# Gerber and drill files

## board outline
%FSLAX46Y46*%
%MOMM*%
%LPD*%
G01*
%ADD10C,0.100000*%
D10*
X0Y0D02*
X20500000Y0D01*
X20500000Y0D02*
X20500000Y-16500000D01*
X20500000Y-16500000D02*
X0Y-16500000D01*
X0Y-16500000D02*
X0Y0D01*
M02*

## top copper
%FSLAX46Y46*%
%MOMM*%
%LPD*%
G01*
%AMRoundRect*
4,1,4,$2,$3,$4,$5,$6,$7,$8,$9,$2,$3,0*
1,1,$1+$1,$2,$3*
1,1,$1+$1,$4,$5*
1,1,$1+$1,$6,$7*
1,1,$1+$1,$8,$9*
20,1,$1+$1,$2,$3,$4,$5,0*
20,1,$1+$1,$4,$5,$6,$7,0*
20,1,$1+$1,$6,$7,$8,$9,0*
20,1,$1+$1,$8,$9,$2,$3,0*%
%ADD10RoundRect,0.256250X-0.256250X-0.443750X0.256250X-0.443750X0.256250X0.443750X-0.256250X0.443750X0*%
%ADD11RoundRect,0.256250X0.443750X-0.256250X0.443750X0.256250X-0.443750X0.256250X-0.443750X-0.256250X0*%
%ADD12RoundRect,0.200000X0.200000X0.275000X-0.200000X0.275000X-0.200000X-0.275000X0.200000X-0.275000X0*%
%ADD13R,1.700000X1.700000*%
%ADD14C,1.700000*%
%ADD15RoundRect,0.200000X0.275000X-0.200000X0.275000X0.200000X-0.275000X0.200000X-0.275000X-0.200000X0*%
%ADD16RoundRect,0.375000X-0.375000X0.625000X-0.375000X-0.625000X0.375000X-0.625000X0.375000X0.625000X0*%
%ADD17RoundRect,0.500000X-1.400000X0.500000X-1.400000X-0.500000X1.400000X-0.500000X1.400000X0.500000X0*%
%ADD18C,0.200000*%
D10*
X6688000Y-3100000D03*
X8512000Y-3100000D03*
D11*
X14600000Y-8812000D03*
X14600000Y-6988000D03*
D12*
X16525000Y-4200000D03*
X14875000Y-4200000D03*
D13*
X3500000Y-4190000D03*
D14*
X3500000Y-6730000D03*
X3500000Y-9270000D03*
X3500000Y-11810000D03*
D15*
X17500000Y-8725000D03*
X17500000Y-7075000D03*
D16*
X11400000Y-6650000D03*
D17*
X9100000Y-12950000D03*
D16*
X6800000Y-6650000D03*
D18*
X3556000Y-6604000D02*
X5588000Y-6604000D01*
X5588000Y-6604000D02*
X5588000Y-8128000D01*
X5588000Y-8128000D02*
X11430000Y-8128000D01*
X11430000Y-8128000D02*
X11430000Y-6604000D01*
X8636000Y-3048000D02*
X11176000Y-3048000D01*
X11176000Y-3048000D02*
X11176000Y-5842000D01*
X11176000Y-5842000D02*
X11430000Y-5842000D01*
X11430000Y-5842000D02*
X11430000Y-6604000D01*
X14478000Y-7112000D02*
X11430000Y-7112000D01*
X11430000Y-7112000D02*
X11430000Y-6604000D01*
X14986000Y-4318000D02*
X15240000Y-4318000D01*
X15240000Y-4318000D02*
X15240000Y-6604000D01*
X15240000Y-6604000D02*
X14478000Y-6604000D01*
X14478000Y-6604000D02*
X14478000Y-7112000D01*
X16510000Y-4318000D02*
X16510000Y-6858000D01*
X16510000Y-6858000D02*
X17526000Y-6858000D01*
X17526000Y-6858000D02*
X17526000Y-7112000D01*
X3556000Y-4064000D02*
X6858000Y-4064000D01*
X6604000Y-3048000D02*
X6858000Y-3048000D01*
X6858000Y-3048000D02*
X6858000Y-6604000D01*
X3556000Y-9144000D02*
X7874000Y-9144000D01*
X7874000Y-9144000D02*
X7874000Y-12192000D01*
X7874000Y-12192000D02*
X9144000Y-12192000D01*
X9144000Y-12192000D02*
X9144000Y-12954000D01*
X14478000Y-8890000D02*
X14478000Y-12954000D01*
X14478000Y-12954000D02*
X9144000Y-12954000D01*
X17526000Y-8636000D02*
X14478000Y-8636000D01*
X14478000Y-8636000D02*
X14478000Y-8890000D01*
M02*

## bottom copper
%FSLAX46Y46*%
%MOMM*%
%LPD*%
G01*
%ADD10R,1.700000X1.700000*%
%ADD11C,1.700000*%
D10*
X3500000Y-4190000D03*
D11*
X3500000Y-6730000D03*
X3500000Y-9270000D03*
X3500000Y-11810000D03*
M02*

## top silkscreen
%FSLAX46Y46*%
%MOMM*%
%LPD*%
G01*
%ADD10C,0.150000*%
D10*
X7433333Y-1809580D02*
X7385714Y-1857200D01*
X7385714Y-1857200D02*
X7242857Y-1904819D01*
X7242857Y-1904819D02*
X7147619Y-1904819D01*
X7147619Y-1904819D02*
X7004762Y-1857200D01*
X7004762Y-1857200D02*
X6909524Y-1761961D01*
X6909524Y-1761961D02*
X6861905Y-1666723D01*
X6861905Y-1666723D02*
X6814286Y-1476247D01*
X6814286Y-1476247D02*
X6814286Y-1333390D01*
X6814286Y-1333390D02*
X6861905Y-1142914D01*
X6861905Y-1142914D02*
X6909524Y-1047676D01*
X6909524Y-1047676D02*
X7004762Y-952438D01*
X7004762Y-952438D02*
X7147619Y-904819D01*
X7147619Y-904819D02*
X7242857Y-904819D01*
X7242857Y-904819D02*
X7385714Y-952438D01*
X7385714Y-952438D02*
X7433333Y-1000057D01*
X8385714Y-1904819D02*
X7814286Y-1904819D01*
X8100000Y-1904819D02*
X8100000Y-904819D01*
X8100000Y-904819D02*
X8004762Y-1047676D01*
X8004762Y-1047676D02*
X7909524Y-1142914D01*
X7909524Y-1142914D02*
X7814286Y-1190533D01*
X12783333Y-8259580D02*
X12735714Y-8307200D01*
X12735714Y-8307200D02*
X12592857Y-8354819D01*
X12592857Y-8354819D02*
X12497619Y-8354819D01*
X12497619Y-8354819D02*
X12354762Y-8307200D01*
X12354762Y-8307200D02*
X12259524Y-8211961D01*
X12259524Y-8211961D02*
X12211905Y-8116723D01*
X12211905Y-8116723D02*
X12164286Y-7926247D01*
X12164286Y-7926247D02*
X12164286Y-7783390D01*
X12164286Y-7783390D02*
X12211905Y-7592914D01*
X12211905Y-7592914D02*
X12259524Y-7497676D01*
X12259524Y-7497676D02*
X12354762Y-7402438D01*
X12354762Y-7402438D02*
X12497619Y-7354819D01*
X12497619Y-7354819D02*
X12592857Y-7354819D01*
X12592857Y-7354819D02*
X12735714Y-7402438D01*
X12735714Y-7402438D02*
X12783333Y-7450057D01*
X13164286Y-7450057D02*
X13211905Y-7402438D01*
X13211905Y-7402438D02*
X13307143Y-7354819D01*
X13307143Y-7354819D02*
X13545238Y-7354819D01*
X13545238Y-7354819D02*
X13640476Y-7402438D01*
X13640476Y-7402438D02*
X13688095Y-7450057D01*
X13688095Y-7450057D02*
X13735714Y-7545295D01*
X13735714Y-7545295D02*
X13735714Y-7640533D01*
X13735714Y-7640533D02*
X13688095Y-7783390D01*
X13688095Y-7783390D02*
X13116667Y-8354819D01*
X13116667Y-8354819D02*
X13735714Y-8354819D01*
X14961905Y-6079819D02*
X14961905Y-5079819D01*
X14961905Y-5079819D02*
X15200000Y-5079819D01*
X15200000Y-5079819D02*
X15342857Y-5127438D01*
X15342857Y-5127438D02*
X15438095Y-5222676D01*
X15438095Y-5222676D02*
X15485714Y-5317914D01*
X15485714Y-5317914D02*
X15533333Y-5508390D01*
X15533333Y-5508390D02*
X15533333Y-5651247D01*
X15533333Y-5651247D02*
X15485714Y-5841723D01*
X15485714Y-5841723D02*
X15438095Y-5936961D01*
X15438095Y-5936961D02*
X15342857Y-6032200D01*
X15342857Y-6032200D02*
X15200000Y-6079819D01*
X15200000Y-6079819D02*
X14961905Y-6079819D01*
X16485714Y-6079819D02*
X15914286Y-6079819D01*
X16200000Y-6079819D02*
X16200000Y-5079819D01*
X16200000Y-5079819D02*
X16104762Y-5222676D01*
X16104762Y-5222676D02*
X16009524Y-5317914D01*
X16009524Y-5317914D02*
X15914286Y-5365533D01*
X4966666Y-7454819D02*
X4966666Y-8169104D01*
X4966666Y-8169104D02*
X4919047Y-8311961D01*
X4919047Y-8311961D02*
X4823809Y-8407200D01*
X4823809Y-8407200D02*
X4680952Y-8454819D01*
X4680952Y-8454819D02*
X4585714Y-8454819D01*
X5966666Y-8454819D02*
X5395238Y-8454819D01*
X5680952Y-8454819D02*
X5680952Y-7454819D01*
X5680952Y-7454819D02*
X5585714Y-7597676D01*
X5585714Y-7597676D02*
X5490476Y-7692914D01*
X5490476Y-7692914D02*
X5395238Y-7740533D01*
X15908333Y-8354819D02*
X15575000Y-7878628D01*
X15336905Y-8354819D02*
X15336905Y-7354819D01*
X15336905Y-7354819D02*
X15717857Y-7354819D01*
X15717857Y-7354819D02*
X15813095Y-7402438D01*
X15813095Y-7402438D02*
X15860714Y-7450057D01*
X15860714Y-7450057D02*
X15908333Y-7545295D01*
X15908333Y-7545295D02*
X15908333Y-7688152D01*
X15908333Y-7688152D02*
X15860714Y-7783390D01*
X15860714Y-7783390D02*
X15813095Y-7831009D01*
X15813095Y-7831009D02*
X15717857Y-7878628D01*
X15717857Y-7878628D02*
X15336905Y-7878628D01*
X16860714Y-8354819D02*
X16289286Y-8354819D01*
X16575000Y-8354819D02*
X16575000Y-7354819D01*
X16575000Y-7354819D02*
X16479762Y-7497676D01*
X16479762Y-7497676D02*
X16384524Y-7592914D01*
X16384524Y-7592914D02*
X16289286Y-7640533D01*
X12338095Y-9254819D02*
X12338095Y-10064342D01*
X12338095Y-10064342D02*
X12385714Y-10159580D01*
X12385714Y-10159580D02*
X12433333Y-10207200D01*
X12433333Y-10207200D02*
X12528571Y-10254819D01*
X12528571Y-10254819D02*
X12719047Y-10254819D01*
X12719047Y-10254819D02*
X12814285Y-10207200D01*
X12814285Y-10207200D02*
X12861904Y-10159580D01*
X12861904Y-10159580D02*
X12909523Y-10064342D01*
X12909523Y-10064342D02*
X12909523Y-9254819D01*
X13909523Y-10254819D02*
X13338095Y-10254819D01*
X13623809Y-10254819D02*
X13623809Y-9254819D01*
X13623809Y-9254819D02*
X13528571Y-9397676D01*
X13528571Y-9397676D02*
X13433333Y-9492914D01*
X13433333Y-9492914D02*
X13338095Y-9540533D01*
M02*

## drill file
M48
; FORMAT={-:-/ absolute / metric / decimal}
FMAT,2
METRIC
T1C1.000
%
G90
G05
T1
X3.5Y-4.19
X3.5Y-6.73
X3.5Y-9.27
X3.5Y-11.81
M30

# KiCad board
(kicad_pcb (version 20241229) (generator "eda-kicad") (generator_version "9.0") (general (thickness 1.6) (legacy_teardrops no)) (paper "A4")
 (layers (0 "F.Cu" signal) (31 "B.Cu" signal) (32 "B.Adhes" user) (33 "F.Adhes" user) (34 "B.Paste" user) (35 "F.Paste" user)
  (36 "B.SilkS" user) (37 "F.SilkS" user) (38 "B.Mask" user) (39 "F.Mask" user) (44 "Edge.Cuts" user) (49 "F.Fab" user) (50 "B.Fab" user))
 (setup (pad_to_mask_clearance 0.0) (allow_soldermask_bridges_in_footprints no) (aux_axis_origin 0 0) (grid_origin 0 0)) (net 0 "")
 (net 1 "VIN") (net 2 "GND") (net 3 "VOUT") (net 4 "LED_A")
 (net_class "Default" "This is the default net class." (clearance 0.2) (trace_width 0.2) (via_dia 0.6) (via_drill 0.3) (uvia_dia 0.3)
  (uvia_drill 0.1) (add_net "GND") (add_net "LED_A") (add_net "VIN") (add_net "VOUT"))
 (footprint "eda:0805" (layer "F.Cu") (at 7.6 3.1 0)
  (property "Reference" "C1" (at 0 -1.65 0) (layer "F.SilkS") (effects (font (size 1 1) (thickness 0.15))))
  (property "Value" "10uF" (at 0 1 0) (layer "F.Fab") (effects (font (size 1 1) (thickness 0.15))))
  (pad "1" smd roundrect (at -0.912 0 0) (size 1.025 1.4) (roundrect_rratio 0.25) (layers "F.Cu" "F.Paste" "F.Mask") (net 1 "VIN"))
  (pad "2" smd roundrect (at 0.912 0 0) (size 1.025 1.4) (roundrect_rratio 0.25) (layers "F.Cu" "F.Paste" "F.Mask") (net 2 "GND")))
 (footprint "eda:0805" (layer "F.Cu") (at 14.6 7.9 -270)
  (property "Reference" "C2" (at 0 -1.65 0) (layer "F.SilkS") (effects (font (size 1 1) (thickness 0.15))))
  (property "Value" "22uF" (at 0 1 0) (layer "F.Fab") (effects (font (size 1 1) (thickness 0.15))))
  (pad "1" smd roundrect (at -0.912 0 -270) (size 1.025 1.4) (roundrect_rratio 0.25) (layers "F.Cu" "F.Paste" "F.Mask") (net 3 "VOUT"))
  (pad "2" smd roundrect (at 0.912 0 -270) (size 1.025 1.4) (roundrect_rratio 0.25) (layers "F.Cu" "F.Paste" "F.Mask") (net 2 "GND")))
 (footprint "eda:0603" (layer "F.Cu") (at 15.7 4.2 -180)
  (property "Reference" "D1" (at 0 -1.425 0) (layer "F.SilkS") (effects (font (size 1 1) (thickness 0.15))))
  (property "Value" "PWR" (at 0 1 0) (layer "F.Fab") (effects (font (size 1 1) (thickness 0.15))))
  (pad "1" smd roundrect (at -0.825 0 -180) (size 0.8 0.95) (roundrect_rratio 0.25) (layers "F.Cu" "F.Paste" "F.Mask") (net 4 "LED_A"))
  (pad "2" smd roundrect (at 0.825 0 -180) (size 0.8 0.95) (roundrect_rratio 0.25) (layers "F.Cu" "F.Paste" "F.Mask") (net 2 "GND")))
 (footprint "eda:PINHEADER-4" (layer "F.Cu") (at 3.5 8 -90)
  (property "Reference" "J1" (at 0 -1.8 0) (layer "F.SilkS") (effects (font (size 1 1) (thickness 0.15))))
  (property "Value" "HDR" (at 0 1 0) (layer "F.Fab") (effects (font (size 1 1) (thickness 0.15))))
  (pad "1" thru_hole rect (at -3.81 0 -90) (size 1.7 1.7) (drill 1) (layers "*.Cu" "*.Mask") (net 1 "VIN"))
  (pad "2" thru_hole circle (at -1.27 0 -90) (size 1.7 1.7) (drill 1) (layers "*.Cu" "*.Mask") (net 2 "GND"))
  (pad "3" thru_hole circle (at 1.27 0 -90) (size 1.7 1.7) (drill 1) (layers "*.Cu" "*.Mask") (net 3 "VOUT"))
  (pad "4" thru_hole circle (at 3.81 0 -90) (size 1.7 1.7) (drill 1) (layers "*.Cu" "*.Mask")))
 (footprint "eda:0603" (layer "F.Cu") (at 17.5 7.9 -270)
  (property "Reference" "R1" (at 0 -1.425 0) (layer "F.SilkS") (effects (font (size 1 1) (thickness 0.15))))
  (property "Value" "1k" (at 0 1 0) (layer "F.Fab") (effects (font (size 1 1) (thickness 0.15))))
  (pad "1" smd roundrect (at -0.825 0 -270) (size 0.8 0.95) (roundrect_rratio 0.25) (layers "F.Cu" "F.Paste" "F.Mask") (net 3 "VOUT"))
  (pad "2" smd roundrect (at 0.825 0 -270) (size 0.8 0.95) (roundrect_rratio 0.25) (layers "F.Cu" "F.Paste" "F.Mask") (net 4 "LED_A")))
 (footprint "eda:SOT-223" (layer "F.Cu") (at 9.1 9.8 -90)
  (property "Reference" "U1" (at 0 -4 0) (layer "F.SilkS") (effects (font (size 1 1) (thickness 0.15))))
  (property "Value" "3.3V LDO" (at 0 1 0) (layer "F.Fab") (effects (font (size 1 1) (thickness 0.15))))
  (pad "1" smd roundrect (at -3.15 -2.3 -90) (size 2 1.5) (roundrect_rratio 0.25) (layers "F.Cu" "F.Paste" "F.Mask") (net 2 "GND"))
  (pad "2" smd roundrect (at 3.15 0 -90) (size 2 3.8) (roundrect_rratio 0.25) (layers "F.Cu" "F.Paste" "F.Mask") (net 3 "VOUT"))
  (pad "3" smd roundrect (at -3.15 2.3 -90) (size 2 1.5) (roundrect_rratio 0.25) (layers "F.Cu" "F.Paste" "F.Mask") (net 1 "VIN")))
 (segment (start 3.556 6.604) (end 5.588 6.604) (width 0.2) (layer "F.Cu") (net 2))
 (segment (start 5.588 6.604) (end 5.588 8.128) (width 0.2) (layer "F.Cu") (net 2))
 (segment (start 5.588 8.128) (end 11.43 8.128) (width 0.2) (layer "F.Cu") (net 2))
 (segment (start 11.43 8.128) (end 11.43 6.604) (width 0.2) (layer "F.Cu") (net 2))
 (segment (start 8.636 3.048) (end 11.176 3.048) (width 0.2) (layer "F.Cu") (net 2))
 (segment (start 11.176 3.048) (end 11.176 5.842) (width 0.2) (layer "F.Cu") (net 2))
 (segment (start 11.176 5.842) (end 11.43 5.842) (width 0.2) (layer "F.Cu") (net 2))
 (segment (start 11.43 5.842) (end 11.43 6.604) (width 0.2) (layer "F.Cu") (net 2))
 (segment (start 14.478 7.112) (end 11.43 7.112) (width 0.2) (layer "F.Cu") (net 2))
 (segment (start 11.43 7.112) (end 11.43 6.604) (width 0.2) (layer "F.Cu") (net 2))
 (segment (start 14.986 4.318) (end 15.24 4.318) (width 0.2) (layer "F.Cu") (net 2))
 (segment (start 15.24 4.318) (end 15.24 6.604) (width 0.2) (layer "F.Cu") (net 2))
 (segment (start 15.24 6.604) (end 14.478 6.604) (width 0.2) (layer "F.Cu") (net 2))
 (segment (start 14.478 6.604) (end 14.478 7.112) (width 0.2) (layer "F.Cu") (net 2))
 (segment (start 16.51 4.318) (end 16.51 6.858) (width 0.2) (layer "F.Cu") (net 4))
 (segment (start 16.51 6.858) (end 17.526 6.858) (width 0.2) (layer "F.Cu") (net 4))
 (segment (start 17.526 6.858) (end 17.526 7.112) (width 0.2) (layer "F.Cu") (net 4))
 (segment (start 3.556 4.064) (end 6.858 4.064) (width 0.2) (layer "F.Cu") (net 1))
 (segment (start 6.604 3.048) (end 6.858 3.048) (width 0.2) (layer "F.Cu") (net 1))
 (segment (start 6.858 3.048) (end 6.858 6.604) (width 0.2) (layer "F.Cu") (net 1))
 (segment (start 3.556 9.144) (end 7.874 9.144) (width 0.2) (layer "F.Cu") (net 3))
 (segment (start 7.874 9.144) (end 7.874 12.192) (width 0.2) (layer "F.Cu") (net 3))
 (segment (start 7.874 12.192) (end 9.144 12.192) (width 0.2) (layer "F.Cu") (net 3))
 (segment (start 9.144 12.192) (end 9.144 12.954) (width 0.2) (layer "F.Cu") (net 3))
 (segment (start 14.478 8.89) (end 14.478 12.954) (width 0.2) (layer "F.Cu") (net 3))
 (segment (start 14.478 12.954) (end 9.144 12.954) (width 0.2) (layer "F.Cu") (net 3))
 (segment (start 17.526 8.636) (end 14.478 8.636) (width 0.2) (layer "F.Cu") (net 3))
 (segment (start 14.478 8.636) (end 14.478 8.89) (width 0.2) (layer "F.Cu") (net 3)) (gr_line (start 0 0) (end 20.5 0) (layer "Edge.Cuts"))
 (gr_line (start 20.5 0) (end 20.5 16.5) (layer "Edge.Cuts")) (gr_line (start 20.5 16.5) (end 0 16.5) (layer "Edge.Cuts"))
 (gr_line (start 0 16.5) (end 0 0) (layer "Edge.Cuts")))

